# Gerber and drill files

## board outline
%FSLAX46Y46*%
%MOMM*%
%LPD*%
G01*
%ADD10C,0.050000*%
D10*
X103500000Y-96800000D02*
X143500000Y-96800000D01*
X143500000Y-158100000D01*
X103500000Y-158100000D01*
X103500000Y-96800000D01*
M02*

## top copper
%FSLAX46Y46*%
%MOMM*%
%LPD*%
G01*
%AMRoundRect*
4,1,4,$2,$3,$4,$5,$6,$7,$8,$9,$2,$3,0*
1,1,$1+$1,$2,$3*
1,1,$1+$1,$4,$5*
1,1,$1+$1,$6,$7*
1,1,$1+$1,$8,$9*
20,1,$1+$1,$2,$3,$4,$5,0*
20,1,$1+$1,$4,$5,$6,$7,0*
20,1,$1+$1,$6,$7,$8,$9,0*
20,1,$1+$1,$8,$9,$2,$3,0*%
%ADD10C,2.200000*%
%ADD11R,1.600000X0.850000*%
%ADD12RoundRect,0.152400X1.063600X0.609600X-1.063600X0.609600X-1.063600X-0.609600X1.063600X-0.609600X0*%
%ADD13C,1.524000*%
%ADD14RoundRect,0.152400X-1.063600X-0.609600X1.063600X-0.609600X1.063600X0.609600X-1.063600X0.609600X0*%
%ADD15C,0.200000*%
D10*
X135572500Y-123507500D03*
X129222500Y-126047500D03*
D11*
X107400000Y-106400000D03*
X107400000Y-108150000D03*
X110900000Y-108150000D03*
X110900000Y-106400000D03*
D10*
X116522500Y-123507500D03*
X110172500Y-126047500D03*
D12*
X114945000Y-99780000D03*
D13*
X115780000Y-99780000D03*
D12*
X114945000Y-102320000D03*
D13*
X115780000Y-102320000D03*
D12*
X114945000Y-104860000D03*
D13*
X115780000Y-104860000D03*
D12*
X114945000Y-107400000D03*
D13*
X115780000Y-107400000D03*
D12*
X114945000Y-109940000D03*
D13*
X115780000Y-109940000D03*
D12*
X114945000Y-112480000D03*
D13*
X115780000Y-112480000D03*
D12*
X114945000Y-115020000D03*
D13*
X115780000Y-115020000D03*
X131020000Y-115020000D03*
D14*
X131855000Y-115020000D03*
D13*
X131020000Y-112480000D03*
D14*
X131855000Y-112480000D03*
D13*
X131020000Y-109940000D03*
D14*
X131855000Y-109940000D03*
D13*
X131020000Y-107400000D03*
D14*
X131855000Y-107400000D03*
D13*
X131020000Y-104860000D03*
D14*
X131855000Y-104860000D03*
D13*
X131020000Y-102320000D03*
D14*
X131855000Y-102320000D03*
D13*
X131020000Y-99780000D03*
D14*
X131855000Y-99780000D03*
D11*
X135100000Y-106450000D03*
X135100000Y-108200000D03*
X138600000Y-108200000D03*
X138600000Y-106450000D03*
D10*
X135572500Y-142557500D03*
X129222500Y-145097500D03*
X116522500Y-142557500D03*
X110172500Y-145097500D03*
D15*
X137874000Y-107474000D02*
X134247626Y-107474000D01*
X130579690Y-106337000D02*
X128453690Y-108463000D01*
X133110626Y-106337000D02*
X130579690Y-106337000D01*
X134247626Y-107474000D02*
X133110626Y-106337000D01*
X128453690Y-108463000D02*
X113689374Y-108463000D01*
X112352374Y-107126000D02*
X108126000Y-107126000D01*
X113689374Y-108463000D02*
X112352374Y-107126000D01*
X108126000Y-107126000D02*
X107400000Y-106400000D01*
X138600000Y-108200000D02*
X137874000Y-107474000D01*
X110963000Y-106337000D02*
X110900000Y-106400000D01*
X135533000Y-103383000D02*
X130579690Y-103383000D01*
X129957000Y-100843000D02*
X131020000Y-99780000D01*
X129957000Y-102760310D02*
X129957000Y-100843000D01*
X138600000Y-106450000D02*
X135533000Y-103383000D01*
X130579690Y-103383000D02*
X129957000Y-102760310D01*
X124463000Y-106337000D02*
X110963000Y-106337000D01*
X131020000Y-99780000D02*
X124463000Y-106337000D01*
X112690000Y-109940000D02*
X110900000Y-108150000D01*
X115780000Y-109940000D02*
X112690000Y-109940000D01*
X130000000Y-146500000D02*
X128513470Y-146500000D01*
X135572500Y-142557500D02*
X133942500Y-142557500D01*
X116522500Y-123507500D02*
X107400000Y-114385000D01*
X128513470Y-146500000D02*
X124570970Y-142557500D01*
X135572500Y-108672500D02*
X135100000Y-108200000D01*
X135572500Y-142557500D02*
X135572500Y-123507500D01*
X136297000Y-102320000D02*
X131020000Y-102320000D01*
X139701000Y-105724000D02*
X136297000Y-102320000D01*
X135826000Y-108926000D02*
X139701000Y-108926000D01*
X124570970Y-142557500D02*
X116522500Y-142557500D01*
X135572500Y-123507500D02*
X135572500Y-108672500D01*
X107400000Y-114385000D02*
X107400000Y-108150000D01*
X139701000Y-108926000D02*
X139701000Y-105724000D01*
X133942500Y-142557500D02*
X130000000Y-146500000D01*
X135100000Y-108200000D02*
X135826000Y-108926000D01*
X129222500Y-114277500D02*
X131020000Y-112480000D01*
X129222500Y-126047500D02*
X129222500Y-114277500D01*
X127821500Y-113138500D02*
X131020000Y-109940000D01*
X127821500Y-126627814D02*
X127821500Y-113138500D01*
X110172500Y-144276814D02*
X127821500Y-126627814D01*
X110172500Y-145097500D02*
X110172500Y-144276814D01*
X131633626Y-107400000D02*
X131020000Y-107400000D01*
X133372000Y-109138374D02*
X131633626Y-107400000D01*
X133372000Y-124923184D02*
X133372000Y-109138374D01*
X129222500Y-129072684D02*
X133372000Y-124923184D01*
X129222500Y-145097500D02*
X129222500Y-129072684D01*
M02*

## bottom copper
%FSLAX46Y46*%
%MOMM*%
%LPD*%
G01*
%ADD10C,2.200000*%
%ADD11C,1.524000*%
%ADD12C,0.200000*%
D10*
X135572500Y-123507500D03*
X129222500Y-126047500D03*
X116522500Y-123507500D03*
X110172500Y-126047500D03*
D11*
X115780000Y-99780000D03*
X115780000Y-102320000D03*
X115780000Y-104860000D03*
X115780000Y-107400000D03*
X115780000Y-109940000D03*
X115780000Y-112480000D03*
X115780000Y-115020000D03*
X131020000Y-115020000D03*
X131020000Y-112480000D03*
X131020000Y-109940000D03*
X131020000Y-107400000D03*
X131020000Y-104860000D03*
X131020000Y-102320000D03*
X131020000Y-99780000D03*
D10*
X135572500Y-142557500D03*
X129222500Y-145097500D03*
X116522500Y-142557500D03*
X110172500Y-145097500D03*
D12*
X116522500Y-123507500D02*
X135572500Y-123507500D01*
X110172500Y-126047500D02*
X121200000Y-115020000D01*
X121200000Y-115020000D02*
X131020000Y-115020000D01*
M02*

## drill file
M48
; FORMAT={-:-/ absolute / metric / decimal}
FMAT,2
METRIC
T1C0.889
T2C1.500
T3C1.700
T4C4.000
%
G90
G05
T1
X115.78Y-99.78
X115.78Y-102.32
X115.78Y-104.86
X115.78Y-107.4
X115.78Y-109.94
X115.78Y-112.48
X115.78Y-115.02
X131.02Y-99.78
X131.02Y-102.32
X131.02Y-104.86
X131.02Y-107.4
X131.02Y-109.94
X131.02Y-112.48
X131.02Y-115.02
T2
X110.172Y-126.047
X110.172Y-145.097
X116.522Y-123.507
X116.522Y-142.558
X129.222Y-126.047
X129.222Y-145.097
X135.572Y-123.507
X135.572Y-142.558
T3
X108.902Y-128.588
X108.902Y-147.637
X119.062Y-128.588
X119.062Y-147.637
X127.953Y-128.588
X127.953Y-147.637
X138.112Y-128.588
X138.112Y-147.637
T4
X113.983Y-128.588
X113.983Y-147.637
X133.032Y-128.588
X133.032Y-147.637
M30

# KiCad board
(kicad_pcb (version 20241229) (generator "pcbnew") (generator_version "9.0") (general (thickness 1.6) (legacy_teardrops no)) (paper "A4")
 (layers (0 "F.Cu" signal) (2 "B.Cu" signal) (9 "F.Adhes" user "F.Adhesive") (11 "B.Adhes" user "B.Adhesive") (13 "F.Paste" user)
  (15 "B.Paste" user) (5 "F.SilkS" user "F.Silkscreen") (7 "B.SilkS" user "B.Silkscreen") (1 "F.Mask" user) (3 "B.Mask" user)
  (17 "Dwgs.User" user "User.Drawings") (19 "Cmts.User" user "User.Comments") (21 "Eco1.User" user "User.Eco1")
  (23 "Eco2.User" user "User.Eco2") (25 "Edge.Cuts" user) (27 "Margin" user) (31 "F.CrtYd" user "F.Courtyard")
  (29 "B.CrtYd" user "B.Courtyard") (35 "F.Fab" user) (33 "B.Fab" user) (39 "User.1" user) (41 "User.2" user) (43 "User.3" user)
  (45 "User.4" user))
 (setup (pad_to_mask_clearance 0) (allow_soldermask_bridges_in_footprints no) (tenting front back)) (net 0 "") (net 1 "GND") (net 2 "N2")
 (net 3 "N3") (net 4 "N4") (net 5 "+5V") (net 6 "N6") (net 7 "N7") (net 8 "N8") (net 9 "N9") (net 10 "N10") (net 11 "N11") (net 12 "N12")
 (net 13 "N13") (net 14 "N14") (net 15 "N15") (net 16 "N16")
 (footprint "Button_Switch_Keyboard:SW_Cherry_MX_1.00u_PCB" (layer "F.Cu") (at 135.5725 123.5075)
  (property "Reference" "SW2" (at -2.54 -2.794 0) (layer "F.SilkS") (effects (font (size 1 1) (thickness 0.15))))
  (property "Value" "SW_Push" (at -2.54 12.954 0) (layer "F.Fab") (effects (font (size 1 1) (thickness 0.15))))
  (pad "" np_thru_hole circle (at -7.62 5.08) (size 1.7 1.7) (drill 1.7) (layers "*.Cu" "*.Mask"))
  (pad "" np_thru_hole circle (at -2.54 5.08) (size 4 4) (drill 4) (layers "*.Cu" "*.Mask"))
  (pad "" np_thru_hole circle (at 2.54 5.08) (size 1.7 1.7) (drill 1.7) (layers "*.Cu" "*.Mask"))
  (pad "1" thru_hole circle (at 0 0) (size 2.2 2.2) (drill 1.5) (layers "*.Cu" "*.Mask") (remove_unused_layers no) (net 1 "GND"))
  (pad "2" thru_hole circle (at -6.35 2.54) (size 2.2 2.2) (drill 1.5) (layers "*.Cu" "*.Mask") (remove_unused_layers no) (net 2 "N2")))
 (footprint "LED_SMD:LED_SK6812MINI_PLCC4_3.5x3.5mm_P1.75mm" (layer "F.Cu") (at 109.15 107.275)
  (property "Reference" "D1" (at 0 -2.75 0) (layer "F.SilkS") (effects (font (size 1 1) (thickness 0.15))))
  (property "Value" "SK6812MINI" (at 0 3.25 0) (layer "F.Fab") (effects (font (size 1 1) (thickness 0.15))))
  (pad "1" smd rect (at -1.75 -0.875) (size 1.6 0.85) (layers "F.Cu" "F.Mask" "F.Paste") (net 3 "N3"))
  (pad "2" smd rect (at -1.75 0.875) (size 1.6 0.85) (layers "F.Cu" "F.Mask" "F.Paste") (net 1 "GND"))
  (pad "3" smd rect (at 1.75 0.875) (size 1.6 0.85) (layers "F.Cu" "F.Mask" "F.Paste") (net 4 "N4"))
  (pad "4" smd rect (at 1.75 -0.875) (size 1.6 0.85) (layers "F.Cu" "F.Mask" "F.Paste") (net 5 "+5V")))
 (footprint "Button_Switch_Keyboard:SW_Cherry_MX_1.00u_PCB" (layer "F.Cu") (at 116.5225 123.5075)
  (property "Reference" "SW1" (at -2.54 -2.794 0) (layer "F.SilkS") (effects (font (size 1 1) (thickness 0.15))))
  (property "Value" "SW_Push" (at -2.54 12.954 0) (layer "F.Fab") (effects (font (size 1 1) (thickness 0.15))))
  (pad "" np_thru_hole circle (at -7.62 5.08) (size 1.7 1.7) (drill 1.7) (layers "*.Cu" "*.Mask"))
  (pad "" np_thru_hole circle (at -2.54 5.08) (size 4 4) (drill 4) (layers "*.Cu" "*.Mask"))
  (pad "" np_thru_hole circle (at 2.54 5.08) (size 1.7 1.7) (drill 1.7) (layers "*.Cu" "*.Mask"))
  (pad "1" thru_hole circle (at 0 0) (size 2.2 2.2) (drill 1.5) (layers "*.Cu" "*.Mask") (remove_unused_layers no) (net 1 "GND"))
  (pad "2" thru_hole circle (at -6.35 2.54) (size 2.2 2.2) (drill 1.5) (layers "*.Cu" "*.Mask") (remove_unused_layers no) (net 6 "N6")))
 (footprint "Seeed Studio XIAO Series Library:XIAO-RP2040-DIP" (layer "F.Cu") (at 123.4 107.4)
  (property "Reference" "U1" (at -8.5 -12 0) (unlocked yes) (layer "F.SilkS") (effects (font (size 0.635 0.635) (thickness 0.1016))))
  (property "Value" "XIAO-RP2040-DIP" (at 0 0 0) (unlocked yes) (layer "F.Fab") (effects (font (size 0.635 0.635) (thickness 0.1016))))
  (pad "1" smd roundrect (at -8.455 -7.62 180) (size 2.432 1.524) (layers "F.Cu" "F.Mask") (roundrect_rratio 0.1) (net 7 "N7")
   (thermal_bridge_angle 45))
  (pad "1" thru_hole circle (at -7.62 -7.62 180) (size 1.524 1.524) (drill 0.889) (layers "*.Cu" "*.Mask") (remove_unused_layers no)
   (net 7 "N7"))
  (pad "2" smd roundrect (at -8.455 -5.08 180) (size 2.432 1.524) (layers "F.Cu" "F.Mask") (roundrect_rratio 0.1) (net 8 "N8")
   (thermal_bridge_angle 45))
  (pad "2" thru_hole circle (at -7.62 -5.08 180) (size 1.524 1.524) (drill 0.889) (layers "*.Cu" "*.Mask") (remove_unused_layers no)
   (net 8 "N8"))
  (pad "3" smd roundrect (at -8.455 -2.54 180) (size 2.432 1.524) (layers "F.Cu" "F.Mask") (roundrect_rratio 0.1) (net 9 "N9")
   (thermal_bridge_angle 45))
  (pad "3" thru_hole circle (at -7.62 -2.54 180) (size 1.524 1.524) (drill 0.889) (layers "*.Cu" "*.Mask") (remove_unused_layers no)
   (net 9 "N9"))
  (pad "4" smd roundrect (at -8.455 0 180) (size 2.432 1.524) (layers "F.Cu" "F.Mask") (roundrect_rratio 0.1) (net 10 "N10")
   (thermal_bridge_angle 45))
  (pad "4" thru_hole circle (at -7.62 0 180) (size 1.524 1.524) (drill 0.889) (layers "*.Cu" "*.Mask") (remove_unused_layers no)
   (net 10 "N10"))
  (pad "5" smd roundrect (at -8.455 2.54 180) (size 2.432 1.524) (layers "F.Cu" "F.Mask") (roundrect_rratio 0.1) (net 4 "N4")
   (thermal_bridge_angle 45))
  (pad "5" thru_hole circle (at -7.62 2.54 180) (size 1.524 1.524) (drill 0.889) (layers "*.Cu" "*.Mask") (remove_unused_layers no)
   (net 4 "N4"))
  (pad "6" smd roundrect (at -8.455 5.08 180) (size 2.432 1.524) (layers "F.Cu" "F.Mask") (roundrect_rratio 0.1) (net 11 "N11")
   (thermal_bridge_angle 45))
  (pad "6" thru_hole circle (at -7.62 5.08 180) (size 1.524 1.524) (drill 0.889) (layers "*.Cu" "*.Mask") (remove_unused_layers no)
   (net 11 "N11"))
  (pad "7" smd roundrect (at -8.455 7.62 180) (size 2.432 1.524) (layers "F.Cu" "F.Mask") (roundrect_rratio 0.1) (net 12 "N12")
   (thermal_bridge_angle 45))
  (pad "7" thru_hole circle (at -7.62 7.62 180) (size 1.524 1.524) (drill 0.889) (layers "*.Cu" "*.Mask") (remove_unused_layers no)
   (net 12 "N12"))
  (pad "8" thru_hole circle (at 7.62 7.62) (size 1.524 1.524) (drill 0.889) (layers "*.Cu" "*.Mask") (remove_unused_layers no) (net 6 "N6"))
  (pad "8" smd roundrect (at 8.455 7.62) (size 2.432 1.524) (layers "F.Cu" "F.Mask") (roundrect_rratio 0.1) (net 6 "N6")
   (thermal_bridge_angle 45))
  (pad "9" thru_hole circle (at 7.62 5.08) (size 1.524 1.524) (drill 0.889) (layers "*.Cu" "*.Mask") (remove_unused_layers no) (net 2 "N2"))
  (pad "9" smd roundrect (at 8.455 5.08) (size 2.432 1.524) (layers "F.Cu" "F.Mask") (roundrect_rratio 0.1) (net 2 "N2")
   (thermal_bridge_angle 45))
  (pad "10" thru_hole circle (at 7.62 2.54) (size 1.524 1.524) (drill 0.889) (layers "*.Cu" "*.Mask") (remove_unused_layers no)
   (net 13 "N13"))
  (pad "10" smd roundrect (at 8.455 2.54) (size 2.432 1.524) (layers "F.Cu" "F.Mask") (roundrect_rratio 0.1) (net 13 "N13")
   (thermal_bridge_angle 45))
  (pad "11" thru_hole circle (at 7.62 0) (size 1.524 1.524) (drill 0.889) (layers "*.Cu" "*.Mask") (remove_unused_layers no) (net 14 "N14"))
  (pad "11" smd roundrect (at 8.455 0) (size 2.432 1.524) (layers "F.Cu" "F.Mask") (roundrect_rratio 0.1) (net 14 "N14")
   (thermal_bridge_angle 45))
  (pad "12" thru_hole circle (at 7.62 -2.54) (size 1.524 1.524) (drill 0.889) (layers "*.Cu" "*.Mask") (remove_unused_layers no)
   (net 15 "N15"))
  (pad "12" smd roundrect (at 8.455 -2.54) (size 2.432 1.524) (layers "F.Cu" "F.Mask") (roundrect_rratio 0.1) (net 15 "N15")
   (thermal_bridge_angle 45))
  (pad "13" thru_hole circle (at 7.62 -5.08) (size 1.524 1.524) (drill 0.889) (layers "*.Cu" "*.Mask") (remove_unused_layers no)
   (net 1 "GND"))
  (pad "13" smd roundrect (at 8.455 -5.08) (size 2.432 1.524) (layers "F.Cu" "F.Mask") (roundrect_rratio 0.1) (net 1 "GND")
   (thermal_bridge_angle 45))
  (pad "14" thru_hole circle (at 7.62 -7.62) (size 1.524 1.524) (drill 0.889) (layers "*.Cu" "*.Mask") (remove_unused_layers no)
   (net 5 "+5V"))
  (pad "14" smd roundrect (at 8.455 -7.62) (size 2.432 1.524) (layers "F.Cu" "F.Mask") (roundrect_rratio 0.1) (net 5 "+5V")
   (thermal_bridge_angle 45)))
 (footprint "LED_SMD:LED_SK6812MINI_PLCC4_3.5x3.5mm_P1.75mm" (layer "F.Cu") (at 136.85 107.325)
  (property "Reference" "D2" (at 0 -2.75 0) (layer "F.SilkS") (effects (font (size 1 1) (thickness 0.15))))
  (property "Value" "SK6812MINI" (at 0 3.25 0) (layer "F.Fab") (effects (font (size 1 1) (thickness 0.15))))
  (pad "1" smd rect (at -1.75 -0.875) (size 1.6 0.85) (layers "F.Cu" "F.Mask" "F.Paste") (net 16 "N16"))
  (pad "2" smd rect (at -1.75 0.875) (size 1.6 0.85) (layers "F.Cu" "F.Mask" "F.Paste") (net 1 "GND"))
  (pad "3" smd rect (at 1.75 0.875) (size 1.6 0.85) (layers "F.Cu" "F.Mask" "F.Paste") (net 3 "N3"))
  (pad "4" smd rect (at 1.75 -0.875) (size 1.6 0.85) (layers "F.Cu" "F.Mask" "F.Paste") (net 5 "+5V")))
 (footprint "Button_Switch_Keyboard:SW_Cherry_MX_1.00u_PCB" (layer "F.Cu") (at 135.5725 142.5575)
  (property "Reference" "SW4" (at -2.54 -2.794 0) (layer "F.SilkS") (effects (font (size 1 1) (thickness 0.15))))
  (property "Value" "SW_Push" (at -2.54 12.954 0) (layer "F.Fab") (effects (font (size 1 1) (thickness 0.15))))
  (pad "" np_thru_hole circle (at -7.62 5.08) (size 1.7 1.7) (drill 1.7) (layers "*.Cu" "*.Mask"))
  (pad "" np_thru_hole circle (at -2.54 5.08) (size 4 4) (drill 4) (layers "*.Cu" "*.Mask"))
  (pad "" np_thru_hole circle (at 2.54 5.08) (size 1.7 1.7) (drill 1.7) (layers "*.Cu" "*.Mask"))
  (pad "1" thru_hole circle (at 0 0) (size 2.2 2.2) (drill 1.5) (layers "*.Cu" "*.Mask") (remove_unused_layers no) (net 1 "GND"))
  (pad "2" thru_hole circle (at -6.35 2.54) (size 2.2 2.2) (drill 1.5) (layers "*.Cu" "*.Mask") (remove_unused_layers no) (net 14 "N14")))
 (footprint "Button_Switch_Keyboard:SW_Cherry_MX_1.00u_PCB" (layer "F.Cu") (at 116.5225 142.5575)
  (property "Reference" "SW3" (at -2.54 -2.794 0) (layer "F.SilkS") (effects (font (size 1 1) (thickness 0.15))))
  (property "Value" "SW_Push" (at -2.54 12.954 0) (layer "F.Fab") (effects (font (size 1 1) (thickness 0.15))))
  (pad "" np_thru_hole circle (at -7.62 5.08) (size 1.7 1.7) (drill 1.7) (layers "*.Cu" "*.Mask"))
  (pad "" np_thru_hole circle (at -2.54 5.08) (size 4 4) (drill 4) (layers "*.Cu" "*.Mask"))
  (pad "" np_thru_hole circle (at 2.54 5.08) (size 1.7 1.7) (drill 1.7) (layers "*.Cu" "*.Mask"))
  (pad "1" thru_hole circle (at 0 0) (size 2.2 2.2) (drill 1.5) (layers "*.Cu" "*.Mask") (remove_unused_layers no) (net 1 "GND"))
  (pad "2" thru_hole circle (at -6.35 2.54) (size 2.2 2.2) (drill 1.5) (layers "*.Cu" "*.Mask") (remove_unused_layers no) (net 13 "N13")))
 (gr_rect (start 103.5 96.8) (end 143.5 158.1) (stroke (width 0.05) (type default)) (fill no) (layer "Edge.Cuts"))
 (segment (start 137.874 107.474) (end 134.247626 107.474) (width 0.2) (layer "F.Cu") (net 3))
 (segment (start 130.57969 106.337) (end 128.45369 108.463) (width 0.2) (layer "F.Cu") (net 3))
 (segment (start 133.110626 106.337) (end 130.57969 106.337) (width 0.2) (layer "F.Cu") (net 3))
 (segment (start 134.247626 107.474) (end 133.110626 106.337) (width 0.2) (layer "F.Cu") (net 3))
 (segment (start 128.45369 108.463) (end 113.689374 108.463) (width 0.2) (layer "F.Cu") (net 3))
 (segment (start 112.352374 107.126) (end 108.126 107.126) (width 0.2) (layer "F.Cu") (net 3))
 (segment (start 113.689374 108.463) (end 112.352374 107.126) (width 0.2) (layer "F.Cu") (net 3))
 (segment (start 108.126 107.126) (end 107.4 106.4) (width 0.2) (layer "F.Cu") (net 3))
 (segment (start 138.6 108.2) (end 137.874 107.474) (width 0.2) (layer "F.Cu") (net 3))
 (segment (start 110.963 106.337) (end 110.9 106.4) (width 0.2) (layer "F.Cu") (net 5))
 (segment (start 135.533 103.383) (end 130.57969 103.383) (width 0.2) (layer "F.Cu") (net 5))
 (segment (start 129.957 100.843) (end 131.02 99.78) (width 0.2) (layer "F.Cu") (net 5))
 (segment (start 129.957 102.76031) (end 129.957 100.843) (width 0.2) (layer "F.Cu") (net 5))
 (segment (start 138.6 106.45) (end 135.533 103.383) (width 0.2) (layer "F.Cu") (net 5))
 (segment (start 130.57969 103.383) (end 129.957 102.76031) (width 0.2) (layer "F.Cu") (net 5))
 (segment (start 124.463 106.337) (end 110.963 106.337) (width 0.2) (layer "F.Cu") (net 5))
 (segment (start 131.02 99.78) (end 124.463 106.337) (width 0.2) (layer "F.Cu") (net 5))
 (segment (start 112.69 109.94) (end 110.9 108.15) (width 0.2) (layer "F.Cu") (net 4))
 (segment (start 115.78 109.94) (end 112.69 109.94) (width 0.2) (layer "F.Cu") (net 4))
 (segment (start 130 146.5) (end 128.51347 146.5) (width 0.2) (layer "F.Cu") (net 1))
 (segment (start 135.5725 142.5575) (end 133.9425 142.5575) (width 0.2) (layer "F.Cu") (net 1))
 (segment (start 116.5225 123.5075) (end 107.4 114.385) (width 0.2) (layer "F.Cu") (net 1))
 (segment (start 128.51347 146.5) (end 124.57097 142.5575) (width 0.2) (layer "F.Cu") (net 1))
 (segment (start 135.5725 108.6725) (end 135.1 108.2) (width 0.2) (layer "F.Cu") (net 1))
 (segment (start 135.5725 142.5575) (end 135.5725 123.5075) (width 0.2) (layer "F.Cu") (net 1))
 (segment (start 136.297 102.32) (end 131.02 102.32) (width 0.2) (layer "F.Cu") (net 1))
 (segment (start 139.701 105.724) (end 136.297 102.32) (width 0.2) (layer "F.Cu") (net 1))
 (segment (start 135.826 108.926) (end 139.701 108.926) (width 0.2) (layer "F.Cu") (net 1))
 (segment (start 124.57097 142.5575) (end 116.5225 142.5575) (width 0.2) (layer "F.Cu") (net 1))
 (segment (start 135.5725 123.5075) (end 135.5725 108.6725) (width 0.2) (layer "F.Cu") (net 1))
 (segment (start 107.4 114.385) (end 107.4 108.15) (width 0.2) (layer "F.Cu") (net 1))
 (segment (start 139.701 108.926) (end 139.701 105.724) (width 0.2) (layer "F.Cu") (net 1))
 (segment (start 133.9425 142.5575) (end 130 146.5) (width 0.2) (layer "F.Cu") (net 1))
 (segment (start 135.1 108.2) (end 135.826 108.926) (width 0.2) (layer "F.Cu") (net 1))
 (segment (start 116.5225 123.5075) (end 135.5725 123.5075) (width 0.2) (layer "B.Cu") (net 1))
 (segment (start 110.1725 126.0475) (end 121.2 115.02) (width 0.2) (layer "B.Cu") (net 6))
 (segment (start 121.2 115.02) (end 131.02 115.02) (width 0.2) (layer "B.Cu") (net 6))
 (segment (start 129.2225 114.2775) (end 131.02 112.48) (width 0.2) (layer "F.Cu") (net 2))
 (segment (start 129.2225 126.0475) (end 129.2225 114.2775) (width 0.2) (layer "F.Cu") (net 2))
 (segment (start 127.8215 113.1385) (end 131.02 109.94) (width 0.2) (layer "F.Cu") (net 13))
 (segment (start 127.8215 126.627814) (end 127.8215 113.1385) (width 0.2) (layer "F.Cu") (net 13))
 (segment (start 110.1725 144.276814) (end 127.8215 126.627814) (width 0.2) (layer "F.Cu") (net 13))
 (segment (start 110.1725 145.0975) (end 110.1725 144.276814) (width 0.2) (layer "F.Cu") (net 13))
 (segment (start 131.633626 107.4) (end 131.02 107.4) (width 0.2) (layer "F.Cu") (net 14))
 (segment (start 133.372 109.138374) (end 131.633626 107.4) (width 0.2) (layer "F.Cu") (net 14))
 (segment (start 133.372 124.923184) (end 133.372 109.138374) (width 0.2) (layer "F.Cu") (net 14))
 (segment (start 129.2225 129.072684) (end 133.372 124.923184) (width 0.2) (layer "F.Cu") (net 14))
 (segment (start 129.2225 145.0975) (end 129.2225 129.072684) (width 0.2) (layer "F.Cu") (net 14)))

